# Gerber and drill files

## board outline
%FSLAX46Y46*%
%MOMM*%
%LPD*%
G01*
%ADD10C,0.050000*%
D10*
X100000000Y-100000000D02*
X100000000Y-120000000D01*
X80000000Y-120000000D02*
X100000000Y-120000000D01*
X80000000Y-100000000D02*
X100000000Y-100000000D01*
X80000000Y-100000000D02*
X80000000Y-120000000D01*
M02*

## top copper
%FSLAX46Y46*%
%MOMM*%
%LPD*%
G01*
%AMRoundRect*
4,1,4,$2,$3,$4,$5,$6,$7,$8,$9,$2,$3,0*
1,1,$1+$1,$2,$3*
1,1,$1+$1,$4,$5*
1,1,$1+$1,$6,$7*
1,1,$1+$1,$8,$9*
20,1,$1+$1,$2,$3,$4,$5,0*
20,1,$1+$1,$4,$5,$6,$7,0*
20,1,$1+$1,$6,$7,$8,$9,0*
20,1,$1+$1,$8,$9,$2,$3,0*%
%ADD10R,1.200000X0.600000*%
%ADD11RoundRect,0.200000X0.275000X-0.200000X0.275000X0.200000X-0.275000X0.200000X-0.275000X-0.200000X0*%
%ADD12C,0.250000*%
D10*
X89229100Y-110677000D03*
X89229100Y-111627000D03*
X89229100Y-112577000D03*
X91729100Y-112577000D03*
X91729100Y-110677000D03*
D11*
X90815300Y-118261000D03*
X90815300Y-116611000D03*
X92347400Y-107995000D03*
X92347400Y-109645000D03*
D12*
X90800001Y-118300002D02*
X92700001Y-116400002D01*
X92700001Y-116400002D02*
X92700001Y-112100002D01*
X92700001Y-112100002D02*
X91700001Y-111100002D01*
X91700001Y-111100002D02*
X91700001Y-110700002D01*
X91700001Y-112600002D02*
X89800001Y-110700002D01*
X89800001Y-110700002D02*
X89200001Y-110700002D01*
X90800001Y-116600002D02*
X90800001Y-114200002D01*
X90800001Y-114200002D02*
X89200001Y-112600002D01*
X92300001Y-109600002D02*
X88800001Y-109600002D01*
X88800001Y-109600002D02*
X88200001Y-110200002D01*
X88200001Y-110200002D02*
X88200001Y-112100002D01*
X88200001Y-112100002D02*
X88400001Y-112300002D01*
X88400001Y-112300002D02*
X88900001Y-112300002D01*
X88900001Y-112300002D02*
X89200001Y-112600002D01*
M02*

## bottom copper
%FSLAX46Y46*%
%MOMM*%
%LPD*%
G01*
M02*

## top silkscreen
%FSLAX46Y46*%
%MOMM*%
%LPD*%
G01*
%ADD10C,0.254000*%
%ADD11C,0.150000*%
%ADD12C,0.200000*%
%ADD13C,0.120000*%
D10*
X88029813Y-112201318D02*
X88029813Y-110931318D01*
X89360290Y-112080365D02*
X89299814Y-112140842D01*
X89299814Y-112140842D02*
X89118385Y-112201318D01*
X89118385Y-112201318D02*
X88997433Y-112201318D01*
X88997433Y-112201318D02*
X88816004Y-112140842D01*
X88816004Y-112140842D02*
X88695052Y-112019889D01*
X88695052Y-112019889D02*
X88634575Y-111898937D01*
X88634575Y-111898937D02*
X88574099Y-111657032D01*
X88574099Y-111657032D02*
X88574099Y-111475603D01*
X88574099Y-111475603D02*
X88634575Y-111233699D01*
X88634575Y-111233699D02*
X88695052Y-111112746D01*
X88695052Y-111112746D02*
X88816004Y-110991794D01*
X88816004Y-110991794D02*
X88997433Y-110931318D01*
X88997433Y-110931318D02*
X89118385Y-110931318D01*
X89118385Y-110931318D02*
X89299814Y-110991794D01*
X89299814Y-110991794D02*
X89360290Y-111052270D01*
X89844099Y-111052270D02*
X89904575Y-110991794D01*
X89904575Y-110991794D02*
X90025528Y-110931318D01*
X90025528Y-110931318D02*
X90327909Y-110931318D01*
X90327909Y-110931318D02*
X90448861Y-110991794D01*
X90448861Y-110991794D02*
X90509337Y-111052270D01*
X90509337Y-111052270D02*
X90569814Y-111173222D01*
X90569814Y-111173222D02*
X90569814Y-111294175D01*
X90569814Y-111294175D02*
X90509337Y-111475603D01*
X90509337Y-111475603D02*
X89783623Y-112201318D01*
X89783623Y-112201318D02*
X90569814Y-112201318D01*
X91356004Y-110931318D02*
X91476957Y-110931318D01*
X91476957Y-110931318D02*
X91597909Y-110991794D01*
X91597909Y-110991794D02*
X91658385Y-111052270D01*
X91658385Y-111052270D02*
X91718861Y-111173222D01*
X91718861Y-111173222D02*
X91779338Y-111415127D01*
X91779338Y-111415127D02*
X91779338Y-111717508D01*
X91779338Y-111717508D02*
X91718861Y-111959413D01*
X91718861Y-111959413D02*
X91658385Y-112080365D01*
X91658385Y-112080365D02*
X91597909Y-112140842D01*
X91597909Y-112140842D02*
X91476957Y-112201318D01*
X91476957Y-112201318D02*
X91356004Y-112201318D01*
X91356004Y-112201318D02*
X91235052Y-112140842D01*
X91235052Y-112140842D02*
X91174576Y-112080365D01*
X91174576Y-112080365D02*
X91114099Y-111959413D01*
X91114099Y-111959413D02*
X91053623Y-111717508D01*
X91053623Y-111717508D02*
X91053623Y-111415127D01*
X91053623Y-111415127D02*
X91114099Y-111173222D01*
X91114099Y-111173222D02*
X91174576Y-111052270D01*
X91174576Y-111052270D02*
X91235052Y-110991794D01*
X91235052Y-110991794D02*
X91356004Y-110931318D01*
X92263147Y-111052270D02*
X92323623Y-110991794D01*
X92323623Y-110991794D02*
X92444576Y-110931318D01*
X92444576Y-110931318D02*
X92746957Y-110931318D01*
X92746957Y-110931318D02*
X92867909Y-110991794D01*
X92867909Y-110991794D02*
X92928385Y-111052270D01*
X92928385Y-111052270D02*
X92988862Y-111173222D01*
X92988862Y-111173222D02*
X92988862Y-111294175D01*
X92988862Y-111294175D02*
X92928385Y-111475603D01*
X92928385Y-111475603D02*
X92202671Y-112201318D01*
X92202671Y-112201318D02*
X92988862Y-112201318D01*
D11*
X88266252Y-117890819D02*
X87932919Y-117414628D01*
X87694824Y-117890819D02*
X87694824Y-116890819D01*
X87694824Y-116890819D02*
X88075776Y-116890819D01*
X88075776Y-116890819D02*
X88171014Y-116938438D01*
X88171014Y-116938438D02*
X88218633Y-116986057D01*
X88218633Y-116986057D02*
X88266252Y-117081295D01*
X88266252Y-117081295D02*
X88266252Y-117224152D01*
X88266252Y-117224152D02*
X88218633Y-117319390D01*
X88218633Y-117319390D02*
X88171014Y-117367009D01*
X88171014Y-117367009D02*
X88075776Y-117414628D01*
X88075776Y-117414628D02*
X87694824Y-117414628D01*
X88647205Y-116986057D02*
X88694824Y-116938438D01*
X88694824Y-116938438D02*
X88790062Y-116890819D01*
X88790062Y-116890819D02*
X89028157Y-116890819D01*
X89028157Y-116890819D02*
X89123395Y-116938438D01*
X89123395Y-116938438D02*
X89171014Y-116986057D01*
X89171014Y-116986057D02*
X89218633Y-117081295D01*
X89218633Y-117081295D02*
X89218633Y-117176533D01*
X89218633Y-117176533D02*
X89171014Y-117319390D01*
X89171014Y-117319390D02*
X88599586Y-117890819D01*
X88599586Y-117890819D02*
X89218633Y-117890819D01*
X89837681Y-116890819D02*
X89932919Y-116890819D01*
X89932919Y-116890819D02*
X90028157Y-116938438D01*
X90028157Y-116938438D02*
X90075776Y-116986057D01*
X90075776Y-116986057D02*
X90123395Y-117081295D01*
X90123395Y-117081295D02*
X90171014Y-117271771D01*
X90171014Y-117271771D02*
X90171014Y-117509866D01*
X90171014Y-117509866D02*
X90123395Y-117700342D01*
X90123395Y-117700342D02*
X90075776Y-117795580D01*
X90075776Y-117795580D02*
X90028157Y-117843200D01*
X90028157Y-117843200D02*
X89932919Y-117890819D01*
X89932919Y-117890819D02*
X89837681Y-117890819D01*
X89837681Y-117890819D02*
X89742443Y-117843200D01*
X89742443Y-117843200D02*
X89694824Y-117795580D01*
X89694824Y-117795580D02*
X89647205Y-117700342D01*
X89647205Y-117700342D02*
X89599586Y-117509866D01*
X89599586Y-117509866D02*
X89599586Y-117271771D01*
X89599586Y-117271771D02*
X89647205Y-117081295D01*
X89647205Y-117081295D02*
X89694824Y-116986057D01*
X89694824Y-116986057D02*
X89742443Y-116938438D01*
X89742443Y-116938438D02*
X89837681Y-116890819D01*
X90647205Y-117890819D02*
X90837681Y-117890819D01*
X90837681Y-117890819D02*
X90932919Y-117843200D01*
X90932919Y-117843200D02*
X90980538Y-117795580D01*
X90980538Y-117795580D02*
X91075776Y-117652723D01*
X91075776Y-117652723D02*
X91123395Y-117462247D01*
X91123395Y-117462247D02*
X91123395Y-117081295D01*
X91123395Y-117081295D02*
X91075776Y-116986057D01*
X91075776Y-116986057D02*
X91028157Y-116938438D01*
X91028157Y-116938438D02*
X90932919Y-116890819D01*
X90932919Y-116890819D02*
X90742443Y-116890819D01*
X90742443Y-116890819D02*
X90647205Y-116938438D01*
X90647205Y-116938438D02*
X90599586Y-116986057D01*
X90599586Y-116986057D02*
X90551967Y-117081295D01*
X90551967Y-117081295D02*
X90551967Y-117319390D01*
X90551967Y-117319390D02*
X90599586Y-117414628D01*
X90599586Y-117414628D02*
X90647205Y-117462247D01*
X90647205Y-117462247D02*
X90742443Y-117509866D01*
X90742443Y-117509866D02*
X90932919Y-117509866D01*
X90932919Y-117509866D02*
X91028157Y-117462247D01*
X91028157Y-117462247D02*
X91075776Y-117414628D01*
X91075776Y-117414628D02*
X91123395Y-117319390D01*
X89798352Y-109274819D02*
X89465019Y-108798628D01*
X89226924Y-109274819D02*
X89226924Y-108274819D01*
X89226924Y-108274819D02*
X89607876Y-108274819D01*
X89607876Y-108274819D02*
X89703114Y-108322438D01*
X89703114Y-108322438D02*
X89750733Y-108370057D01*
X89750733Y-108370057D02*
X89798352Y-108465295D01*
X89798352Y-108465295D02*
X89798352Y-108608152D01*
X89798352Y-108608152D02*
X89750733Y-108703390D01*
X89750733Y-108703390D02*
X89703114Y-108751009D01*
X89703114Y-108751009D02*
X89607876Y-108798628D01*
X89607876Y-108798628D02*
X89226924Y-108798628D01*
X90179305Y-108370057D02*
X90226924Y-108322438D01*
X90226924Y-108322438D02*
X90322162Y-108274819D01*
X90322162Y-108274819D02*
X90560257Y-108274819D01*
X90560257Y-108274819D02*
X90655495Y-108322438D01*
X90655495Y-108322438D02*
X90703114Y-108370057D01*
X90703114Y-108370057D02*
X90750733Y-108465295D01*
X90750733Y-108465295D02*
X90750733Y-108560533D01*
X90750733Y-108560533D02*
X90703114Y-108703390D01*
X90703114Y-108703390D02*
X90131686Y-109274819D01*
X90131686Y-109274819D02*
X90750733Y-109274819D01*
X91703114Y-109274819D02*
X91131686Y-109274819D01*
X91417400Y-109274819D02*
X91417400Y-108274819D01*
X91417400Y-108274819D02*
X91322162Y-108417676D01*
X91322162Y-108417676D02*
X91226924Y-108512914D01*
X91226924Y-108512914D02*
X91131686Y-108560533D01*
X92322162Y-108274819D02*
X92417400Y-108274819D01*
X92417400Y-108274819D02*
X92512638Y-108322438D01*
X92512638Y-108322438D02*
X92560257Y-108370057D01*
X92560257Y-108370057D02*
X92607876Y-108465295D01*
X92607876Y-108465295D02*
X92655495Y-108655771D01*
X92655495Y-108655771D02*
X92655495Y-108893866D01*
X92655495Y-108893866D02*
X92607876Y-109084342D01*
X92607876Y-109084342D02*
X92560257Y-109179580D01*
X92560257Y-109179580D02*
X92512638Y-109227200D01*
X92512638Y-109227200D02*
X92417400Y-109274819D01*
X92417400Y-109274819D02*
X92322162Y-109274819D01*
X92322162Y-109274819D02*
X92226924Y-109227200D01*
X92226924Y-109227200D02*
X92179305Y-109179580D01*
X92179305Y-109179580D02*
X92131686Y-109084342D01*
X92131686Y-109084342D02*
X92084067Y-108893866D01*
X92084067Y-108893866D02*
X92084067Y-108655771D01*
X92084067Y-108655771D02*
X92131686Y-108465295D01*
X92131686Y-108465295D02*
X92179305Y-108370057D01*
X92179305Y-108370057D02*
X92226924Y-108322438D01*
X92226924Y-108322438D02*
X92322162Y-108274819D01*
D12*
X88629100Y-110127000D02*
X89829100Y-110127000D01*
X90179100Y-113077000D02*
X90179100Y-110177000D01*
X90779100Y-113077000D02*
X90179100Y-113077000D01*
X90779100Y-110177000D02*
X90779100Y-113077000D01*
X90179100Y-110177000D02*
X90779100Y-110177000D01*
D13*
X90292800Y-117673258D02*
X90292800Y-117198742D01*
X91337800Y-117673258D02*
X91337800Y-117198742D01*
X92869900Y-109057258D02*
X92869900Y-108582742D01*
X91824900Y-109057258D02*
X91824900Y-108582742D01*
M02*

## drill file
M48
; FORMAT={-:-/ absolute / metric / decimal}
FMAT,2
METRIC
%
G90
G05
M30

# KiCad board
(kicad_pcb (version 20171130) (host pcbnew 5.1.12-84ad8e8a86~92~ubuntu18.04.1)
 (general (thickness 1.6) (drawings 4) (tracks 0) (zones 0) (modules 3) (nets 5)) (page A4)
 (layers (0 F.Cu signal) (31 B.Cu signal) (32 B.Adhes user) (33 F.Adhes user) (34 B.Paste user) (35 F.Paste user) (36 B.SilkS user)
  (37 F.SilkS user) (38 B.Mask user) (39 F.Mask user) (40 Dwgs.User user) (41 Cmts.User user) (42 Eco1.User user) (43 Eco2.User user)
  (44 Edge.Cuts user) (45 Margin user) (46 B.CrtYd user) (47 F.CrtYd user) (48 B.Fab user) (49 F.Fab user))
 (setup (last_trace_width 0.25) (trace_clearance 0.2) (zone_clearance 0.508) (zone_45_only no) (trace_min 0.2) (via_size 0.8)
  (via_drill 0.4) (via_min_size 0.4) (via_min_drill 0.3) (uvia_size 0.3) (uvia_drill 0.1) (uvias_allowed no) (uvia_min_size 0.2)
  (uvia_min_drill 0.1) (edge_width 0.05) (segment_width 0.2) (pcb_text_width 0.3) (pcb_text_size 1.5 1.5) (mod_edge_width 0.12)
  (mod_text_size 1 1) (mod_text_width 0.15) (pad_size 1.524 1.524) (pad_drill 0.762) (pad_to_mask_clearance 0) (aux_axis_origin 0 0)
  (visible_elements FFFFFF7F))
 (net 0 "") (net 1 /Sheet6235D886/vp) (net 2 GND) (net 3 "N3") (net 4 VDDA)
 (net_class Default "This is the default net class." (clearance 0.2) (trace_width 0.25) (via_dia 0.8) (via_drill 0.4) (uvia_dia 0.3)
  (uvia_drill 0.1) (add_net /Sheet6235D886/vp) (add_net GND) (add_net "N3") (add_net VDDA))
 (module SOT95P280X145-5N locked (layer F.Cu) (at 90.479100 111.627000)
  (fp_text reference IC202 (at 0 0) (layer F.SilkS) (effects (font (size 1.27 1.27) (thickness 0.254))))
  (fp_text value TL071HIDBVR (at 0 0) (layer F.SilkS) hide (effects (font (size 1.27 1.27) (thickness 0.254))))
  (fp_line (start -1.85 -1.5) (end -0.65 -1.5) (layer F.SilkS) (width 0.2))
  (fp_line (start -0.3 1.45) (end -0.3 -1.45) (layer F.SilkS) (width 0.2))
  (fp_line (start 0.3 1.45) (end -0.3 1.45) (layer F.SilkS) (width 0.2))
  (fp_line (start 0.3 -1.45) (end 0.3 1.45) (layer F.SilkS) (width 0.2))
  (fp_line (start -0.3 -1.45) (end 0.3 -1.45) (layer F.SilkS) (width 0.2))
  (pad 1 smd rect (at -1.25 -0.95 90.000000) (size 0.6 1.2) (layers F.Cu F.Mask F.Paste) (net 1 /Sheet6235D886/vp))
  (pad 2 smd rect (at -1.25 0 90.000000) (size 0.6 1.2) (layers F.Cu F.Mask F.Paste) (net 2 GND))
  (pad 3 smd rect (at -1.25 0.95 90.000000) (size 0.6 1.2) (layers F.Cu F.Mask F.Paste) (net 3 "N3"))
  (pad 4 smd rect (at 1.25 0.95 90.000000) (size 0.6 1.2) (layers F.Cu F.Mask F.Paste) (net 1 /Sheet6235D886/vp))
  (pad 5 smd rect (at 1.25 -0.95 90.000000) (size 0.6 1.2) (layers F.Cu F.Mask F.Paste) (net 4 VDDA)))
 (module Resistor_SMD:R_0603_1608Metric (layer F.Cu) (at 90.815300 117.436000 90.000000)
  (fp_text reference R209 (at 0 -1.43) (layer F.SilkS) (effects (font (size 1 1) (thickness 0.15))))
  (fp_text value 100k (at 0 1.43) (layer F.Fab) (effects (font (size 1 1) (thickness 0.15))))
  (fp_line (start -0.237258 -0.5225) (end 0.237258 -0.5225) (layer F.SilkS) (width 0.12))
  (fp_line (start -0.237258 0.5225) (end 0.237258 0.5225) (layer F.SilkS) (width 0.12))
  (pad 1 smd roundrect (at -0.825 0 90.000000) (size 0.8 0.95) (layers F.Cu F.Mask F.Paste) (roundrect_rratio 0.25) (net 4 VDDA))
  (pad 2 smd roundrect (at 0.825 0 90.000000) (size 0.8 0.95) (layers F.Cu F.Mask F.Paste) (roundrect_rratio 0.25) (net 3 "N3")))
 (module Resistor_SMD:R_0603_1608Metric (layer F.Cu) (at 92.347400 108.820000 90.000000)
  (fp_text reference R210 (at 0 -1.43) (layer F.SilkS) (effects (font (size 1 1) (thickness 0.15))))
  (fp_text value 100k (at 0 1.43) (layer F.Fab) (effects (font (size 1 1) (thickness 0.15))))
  (fp_line (start -0.237258 0.5225) (end 0.237258 0.5225) (layer F.SilkS) (width 0.12))
  (fp_line (start -0.237258 -0.5225) (end 0.237258 -0.5225) (layer F.SilkS) (width 0.12))
  (pad 2 smd roundrect (at 0.825 0 90.000000) (size 0.8 0.95) (layers F.Cu F.Mask F.Paste) (roundrect_rratio 0.25) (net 2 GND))
  (pad 1 smd roundrect (at -0.825 0 90.000000) (size 0.8 0.95) (layers F.Cu F.Mask F.Paste) (roundrect_rratio 0.25) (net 3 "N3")))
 (gr_line (start 100 100) (end 100 120) (layer Edge.Cuts) (width 0.05))
 (gr_line (start 80 120) (end 100 120) (layer Edge.Cuts) (width 0.05))
 (gr_line (start 80 100) (end 100 100) (layer Edge.Cuts) (width 0.05))
 (gr_line (start 80 100) (end 80 120) (layer Edge.Cuts) (width 0.05))
 (segment (start 90.800001 118.300002) (end 92.700001 116.400002) (width 0.250000) (layer F.Cu) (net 4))
 (segment (start 92.700001 116.400002) (end 92.700001 112.100002) (width 0.250000) (layer F.Cu) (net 4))
 (segment (start 92.700001 112.100002) (end 91.700001 111.100002) (width 0.250000) (layer F.Cu) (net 4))
 (segment (start 91.700001 111.100002) (end 91.700001 110.700002) (width 0.250000) (layer F.Cu) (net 4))
 (segment (start 91.700001 112.600002) (end 89.800001 110.700002) (width 0.250000) (layer F.Cu) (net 1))
 (segment (start 89.800001 110.700002) (end 89.200001 110.700002) (width 0.250000) (layer F.Cu) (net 1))
 (segment (start 90.800001 116.600002) (end 90.800001 114.200002) (width 0.250000) (layer F.Cu) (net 3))
 (segment (start 90.800001 114.200002) (end 89.200001 112.600002) (width 0.250000) (layer F.Cu) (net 3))
 (segment (start 92.300001 109.600002) (end 88.800001 109.600002) (width 0.250000) (layer F.Cu) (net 3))
 (segment (start 88.800001 109.600002) (end 88.200001 110.200002) (width 0.250000) (layer F.Cu) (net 3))
 (segment (start 88.200001 110.200002) (end 88.200001 112.100002) (width 0.250000) (layer F.Cu) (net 3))
 (segment (start 88.200001 112.100002) (end 88.400001 112.300002) (width 0.250000) (layer F.Cu) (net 3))
 (segment (start 88.400001 112.300002) (end 88.900001 112.300002) (width 0.250000) (layer F.Cu) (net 3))
 (segment (start 88.900001 112.300002) (end 89.200001 112.600002) (width 0.250000) (layer F.Cu) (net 3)))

